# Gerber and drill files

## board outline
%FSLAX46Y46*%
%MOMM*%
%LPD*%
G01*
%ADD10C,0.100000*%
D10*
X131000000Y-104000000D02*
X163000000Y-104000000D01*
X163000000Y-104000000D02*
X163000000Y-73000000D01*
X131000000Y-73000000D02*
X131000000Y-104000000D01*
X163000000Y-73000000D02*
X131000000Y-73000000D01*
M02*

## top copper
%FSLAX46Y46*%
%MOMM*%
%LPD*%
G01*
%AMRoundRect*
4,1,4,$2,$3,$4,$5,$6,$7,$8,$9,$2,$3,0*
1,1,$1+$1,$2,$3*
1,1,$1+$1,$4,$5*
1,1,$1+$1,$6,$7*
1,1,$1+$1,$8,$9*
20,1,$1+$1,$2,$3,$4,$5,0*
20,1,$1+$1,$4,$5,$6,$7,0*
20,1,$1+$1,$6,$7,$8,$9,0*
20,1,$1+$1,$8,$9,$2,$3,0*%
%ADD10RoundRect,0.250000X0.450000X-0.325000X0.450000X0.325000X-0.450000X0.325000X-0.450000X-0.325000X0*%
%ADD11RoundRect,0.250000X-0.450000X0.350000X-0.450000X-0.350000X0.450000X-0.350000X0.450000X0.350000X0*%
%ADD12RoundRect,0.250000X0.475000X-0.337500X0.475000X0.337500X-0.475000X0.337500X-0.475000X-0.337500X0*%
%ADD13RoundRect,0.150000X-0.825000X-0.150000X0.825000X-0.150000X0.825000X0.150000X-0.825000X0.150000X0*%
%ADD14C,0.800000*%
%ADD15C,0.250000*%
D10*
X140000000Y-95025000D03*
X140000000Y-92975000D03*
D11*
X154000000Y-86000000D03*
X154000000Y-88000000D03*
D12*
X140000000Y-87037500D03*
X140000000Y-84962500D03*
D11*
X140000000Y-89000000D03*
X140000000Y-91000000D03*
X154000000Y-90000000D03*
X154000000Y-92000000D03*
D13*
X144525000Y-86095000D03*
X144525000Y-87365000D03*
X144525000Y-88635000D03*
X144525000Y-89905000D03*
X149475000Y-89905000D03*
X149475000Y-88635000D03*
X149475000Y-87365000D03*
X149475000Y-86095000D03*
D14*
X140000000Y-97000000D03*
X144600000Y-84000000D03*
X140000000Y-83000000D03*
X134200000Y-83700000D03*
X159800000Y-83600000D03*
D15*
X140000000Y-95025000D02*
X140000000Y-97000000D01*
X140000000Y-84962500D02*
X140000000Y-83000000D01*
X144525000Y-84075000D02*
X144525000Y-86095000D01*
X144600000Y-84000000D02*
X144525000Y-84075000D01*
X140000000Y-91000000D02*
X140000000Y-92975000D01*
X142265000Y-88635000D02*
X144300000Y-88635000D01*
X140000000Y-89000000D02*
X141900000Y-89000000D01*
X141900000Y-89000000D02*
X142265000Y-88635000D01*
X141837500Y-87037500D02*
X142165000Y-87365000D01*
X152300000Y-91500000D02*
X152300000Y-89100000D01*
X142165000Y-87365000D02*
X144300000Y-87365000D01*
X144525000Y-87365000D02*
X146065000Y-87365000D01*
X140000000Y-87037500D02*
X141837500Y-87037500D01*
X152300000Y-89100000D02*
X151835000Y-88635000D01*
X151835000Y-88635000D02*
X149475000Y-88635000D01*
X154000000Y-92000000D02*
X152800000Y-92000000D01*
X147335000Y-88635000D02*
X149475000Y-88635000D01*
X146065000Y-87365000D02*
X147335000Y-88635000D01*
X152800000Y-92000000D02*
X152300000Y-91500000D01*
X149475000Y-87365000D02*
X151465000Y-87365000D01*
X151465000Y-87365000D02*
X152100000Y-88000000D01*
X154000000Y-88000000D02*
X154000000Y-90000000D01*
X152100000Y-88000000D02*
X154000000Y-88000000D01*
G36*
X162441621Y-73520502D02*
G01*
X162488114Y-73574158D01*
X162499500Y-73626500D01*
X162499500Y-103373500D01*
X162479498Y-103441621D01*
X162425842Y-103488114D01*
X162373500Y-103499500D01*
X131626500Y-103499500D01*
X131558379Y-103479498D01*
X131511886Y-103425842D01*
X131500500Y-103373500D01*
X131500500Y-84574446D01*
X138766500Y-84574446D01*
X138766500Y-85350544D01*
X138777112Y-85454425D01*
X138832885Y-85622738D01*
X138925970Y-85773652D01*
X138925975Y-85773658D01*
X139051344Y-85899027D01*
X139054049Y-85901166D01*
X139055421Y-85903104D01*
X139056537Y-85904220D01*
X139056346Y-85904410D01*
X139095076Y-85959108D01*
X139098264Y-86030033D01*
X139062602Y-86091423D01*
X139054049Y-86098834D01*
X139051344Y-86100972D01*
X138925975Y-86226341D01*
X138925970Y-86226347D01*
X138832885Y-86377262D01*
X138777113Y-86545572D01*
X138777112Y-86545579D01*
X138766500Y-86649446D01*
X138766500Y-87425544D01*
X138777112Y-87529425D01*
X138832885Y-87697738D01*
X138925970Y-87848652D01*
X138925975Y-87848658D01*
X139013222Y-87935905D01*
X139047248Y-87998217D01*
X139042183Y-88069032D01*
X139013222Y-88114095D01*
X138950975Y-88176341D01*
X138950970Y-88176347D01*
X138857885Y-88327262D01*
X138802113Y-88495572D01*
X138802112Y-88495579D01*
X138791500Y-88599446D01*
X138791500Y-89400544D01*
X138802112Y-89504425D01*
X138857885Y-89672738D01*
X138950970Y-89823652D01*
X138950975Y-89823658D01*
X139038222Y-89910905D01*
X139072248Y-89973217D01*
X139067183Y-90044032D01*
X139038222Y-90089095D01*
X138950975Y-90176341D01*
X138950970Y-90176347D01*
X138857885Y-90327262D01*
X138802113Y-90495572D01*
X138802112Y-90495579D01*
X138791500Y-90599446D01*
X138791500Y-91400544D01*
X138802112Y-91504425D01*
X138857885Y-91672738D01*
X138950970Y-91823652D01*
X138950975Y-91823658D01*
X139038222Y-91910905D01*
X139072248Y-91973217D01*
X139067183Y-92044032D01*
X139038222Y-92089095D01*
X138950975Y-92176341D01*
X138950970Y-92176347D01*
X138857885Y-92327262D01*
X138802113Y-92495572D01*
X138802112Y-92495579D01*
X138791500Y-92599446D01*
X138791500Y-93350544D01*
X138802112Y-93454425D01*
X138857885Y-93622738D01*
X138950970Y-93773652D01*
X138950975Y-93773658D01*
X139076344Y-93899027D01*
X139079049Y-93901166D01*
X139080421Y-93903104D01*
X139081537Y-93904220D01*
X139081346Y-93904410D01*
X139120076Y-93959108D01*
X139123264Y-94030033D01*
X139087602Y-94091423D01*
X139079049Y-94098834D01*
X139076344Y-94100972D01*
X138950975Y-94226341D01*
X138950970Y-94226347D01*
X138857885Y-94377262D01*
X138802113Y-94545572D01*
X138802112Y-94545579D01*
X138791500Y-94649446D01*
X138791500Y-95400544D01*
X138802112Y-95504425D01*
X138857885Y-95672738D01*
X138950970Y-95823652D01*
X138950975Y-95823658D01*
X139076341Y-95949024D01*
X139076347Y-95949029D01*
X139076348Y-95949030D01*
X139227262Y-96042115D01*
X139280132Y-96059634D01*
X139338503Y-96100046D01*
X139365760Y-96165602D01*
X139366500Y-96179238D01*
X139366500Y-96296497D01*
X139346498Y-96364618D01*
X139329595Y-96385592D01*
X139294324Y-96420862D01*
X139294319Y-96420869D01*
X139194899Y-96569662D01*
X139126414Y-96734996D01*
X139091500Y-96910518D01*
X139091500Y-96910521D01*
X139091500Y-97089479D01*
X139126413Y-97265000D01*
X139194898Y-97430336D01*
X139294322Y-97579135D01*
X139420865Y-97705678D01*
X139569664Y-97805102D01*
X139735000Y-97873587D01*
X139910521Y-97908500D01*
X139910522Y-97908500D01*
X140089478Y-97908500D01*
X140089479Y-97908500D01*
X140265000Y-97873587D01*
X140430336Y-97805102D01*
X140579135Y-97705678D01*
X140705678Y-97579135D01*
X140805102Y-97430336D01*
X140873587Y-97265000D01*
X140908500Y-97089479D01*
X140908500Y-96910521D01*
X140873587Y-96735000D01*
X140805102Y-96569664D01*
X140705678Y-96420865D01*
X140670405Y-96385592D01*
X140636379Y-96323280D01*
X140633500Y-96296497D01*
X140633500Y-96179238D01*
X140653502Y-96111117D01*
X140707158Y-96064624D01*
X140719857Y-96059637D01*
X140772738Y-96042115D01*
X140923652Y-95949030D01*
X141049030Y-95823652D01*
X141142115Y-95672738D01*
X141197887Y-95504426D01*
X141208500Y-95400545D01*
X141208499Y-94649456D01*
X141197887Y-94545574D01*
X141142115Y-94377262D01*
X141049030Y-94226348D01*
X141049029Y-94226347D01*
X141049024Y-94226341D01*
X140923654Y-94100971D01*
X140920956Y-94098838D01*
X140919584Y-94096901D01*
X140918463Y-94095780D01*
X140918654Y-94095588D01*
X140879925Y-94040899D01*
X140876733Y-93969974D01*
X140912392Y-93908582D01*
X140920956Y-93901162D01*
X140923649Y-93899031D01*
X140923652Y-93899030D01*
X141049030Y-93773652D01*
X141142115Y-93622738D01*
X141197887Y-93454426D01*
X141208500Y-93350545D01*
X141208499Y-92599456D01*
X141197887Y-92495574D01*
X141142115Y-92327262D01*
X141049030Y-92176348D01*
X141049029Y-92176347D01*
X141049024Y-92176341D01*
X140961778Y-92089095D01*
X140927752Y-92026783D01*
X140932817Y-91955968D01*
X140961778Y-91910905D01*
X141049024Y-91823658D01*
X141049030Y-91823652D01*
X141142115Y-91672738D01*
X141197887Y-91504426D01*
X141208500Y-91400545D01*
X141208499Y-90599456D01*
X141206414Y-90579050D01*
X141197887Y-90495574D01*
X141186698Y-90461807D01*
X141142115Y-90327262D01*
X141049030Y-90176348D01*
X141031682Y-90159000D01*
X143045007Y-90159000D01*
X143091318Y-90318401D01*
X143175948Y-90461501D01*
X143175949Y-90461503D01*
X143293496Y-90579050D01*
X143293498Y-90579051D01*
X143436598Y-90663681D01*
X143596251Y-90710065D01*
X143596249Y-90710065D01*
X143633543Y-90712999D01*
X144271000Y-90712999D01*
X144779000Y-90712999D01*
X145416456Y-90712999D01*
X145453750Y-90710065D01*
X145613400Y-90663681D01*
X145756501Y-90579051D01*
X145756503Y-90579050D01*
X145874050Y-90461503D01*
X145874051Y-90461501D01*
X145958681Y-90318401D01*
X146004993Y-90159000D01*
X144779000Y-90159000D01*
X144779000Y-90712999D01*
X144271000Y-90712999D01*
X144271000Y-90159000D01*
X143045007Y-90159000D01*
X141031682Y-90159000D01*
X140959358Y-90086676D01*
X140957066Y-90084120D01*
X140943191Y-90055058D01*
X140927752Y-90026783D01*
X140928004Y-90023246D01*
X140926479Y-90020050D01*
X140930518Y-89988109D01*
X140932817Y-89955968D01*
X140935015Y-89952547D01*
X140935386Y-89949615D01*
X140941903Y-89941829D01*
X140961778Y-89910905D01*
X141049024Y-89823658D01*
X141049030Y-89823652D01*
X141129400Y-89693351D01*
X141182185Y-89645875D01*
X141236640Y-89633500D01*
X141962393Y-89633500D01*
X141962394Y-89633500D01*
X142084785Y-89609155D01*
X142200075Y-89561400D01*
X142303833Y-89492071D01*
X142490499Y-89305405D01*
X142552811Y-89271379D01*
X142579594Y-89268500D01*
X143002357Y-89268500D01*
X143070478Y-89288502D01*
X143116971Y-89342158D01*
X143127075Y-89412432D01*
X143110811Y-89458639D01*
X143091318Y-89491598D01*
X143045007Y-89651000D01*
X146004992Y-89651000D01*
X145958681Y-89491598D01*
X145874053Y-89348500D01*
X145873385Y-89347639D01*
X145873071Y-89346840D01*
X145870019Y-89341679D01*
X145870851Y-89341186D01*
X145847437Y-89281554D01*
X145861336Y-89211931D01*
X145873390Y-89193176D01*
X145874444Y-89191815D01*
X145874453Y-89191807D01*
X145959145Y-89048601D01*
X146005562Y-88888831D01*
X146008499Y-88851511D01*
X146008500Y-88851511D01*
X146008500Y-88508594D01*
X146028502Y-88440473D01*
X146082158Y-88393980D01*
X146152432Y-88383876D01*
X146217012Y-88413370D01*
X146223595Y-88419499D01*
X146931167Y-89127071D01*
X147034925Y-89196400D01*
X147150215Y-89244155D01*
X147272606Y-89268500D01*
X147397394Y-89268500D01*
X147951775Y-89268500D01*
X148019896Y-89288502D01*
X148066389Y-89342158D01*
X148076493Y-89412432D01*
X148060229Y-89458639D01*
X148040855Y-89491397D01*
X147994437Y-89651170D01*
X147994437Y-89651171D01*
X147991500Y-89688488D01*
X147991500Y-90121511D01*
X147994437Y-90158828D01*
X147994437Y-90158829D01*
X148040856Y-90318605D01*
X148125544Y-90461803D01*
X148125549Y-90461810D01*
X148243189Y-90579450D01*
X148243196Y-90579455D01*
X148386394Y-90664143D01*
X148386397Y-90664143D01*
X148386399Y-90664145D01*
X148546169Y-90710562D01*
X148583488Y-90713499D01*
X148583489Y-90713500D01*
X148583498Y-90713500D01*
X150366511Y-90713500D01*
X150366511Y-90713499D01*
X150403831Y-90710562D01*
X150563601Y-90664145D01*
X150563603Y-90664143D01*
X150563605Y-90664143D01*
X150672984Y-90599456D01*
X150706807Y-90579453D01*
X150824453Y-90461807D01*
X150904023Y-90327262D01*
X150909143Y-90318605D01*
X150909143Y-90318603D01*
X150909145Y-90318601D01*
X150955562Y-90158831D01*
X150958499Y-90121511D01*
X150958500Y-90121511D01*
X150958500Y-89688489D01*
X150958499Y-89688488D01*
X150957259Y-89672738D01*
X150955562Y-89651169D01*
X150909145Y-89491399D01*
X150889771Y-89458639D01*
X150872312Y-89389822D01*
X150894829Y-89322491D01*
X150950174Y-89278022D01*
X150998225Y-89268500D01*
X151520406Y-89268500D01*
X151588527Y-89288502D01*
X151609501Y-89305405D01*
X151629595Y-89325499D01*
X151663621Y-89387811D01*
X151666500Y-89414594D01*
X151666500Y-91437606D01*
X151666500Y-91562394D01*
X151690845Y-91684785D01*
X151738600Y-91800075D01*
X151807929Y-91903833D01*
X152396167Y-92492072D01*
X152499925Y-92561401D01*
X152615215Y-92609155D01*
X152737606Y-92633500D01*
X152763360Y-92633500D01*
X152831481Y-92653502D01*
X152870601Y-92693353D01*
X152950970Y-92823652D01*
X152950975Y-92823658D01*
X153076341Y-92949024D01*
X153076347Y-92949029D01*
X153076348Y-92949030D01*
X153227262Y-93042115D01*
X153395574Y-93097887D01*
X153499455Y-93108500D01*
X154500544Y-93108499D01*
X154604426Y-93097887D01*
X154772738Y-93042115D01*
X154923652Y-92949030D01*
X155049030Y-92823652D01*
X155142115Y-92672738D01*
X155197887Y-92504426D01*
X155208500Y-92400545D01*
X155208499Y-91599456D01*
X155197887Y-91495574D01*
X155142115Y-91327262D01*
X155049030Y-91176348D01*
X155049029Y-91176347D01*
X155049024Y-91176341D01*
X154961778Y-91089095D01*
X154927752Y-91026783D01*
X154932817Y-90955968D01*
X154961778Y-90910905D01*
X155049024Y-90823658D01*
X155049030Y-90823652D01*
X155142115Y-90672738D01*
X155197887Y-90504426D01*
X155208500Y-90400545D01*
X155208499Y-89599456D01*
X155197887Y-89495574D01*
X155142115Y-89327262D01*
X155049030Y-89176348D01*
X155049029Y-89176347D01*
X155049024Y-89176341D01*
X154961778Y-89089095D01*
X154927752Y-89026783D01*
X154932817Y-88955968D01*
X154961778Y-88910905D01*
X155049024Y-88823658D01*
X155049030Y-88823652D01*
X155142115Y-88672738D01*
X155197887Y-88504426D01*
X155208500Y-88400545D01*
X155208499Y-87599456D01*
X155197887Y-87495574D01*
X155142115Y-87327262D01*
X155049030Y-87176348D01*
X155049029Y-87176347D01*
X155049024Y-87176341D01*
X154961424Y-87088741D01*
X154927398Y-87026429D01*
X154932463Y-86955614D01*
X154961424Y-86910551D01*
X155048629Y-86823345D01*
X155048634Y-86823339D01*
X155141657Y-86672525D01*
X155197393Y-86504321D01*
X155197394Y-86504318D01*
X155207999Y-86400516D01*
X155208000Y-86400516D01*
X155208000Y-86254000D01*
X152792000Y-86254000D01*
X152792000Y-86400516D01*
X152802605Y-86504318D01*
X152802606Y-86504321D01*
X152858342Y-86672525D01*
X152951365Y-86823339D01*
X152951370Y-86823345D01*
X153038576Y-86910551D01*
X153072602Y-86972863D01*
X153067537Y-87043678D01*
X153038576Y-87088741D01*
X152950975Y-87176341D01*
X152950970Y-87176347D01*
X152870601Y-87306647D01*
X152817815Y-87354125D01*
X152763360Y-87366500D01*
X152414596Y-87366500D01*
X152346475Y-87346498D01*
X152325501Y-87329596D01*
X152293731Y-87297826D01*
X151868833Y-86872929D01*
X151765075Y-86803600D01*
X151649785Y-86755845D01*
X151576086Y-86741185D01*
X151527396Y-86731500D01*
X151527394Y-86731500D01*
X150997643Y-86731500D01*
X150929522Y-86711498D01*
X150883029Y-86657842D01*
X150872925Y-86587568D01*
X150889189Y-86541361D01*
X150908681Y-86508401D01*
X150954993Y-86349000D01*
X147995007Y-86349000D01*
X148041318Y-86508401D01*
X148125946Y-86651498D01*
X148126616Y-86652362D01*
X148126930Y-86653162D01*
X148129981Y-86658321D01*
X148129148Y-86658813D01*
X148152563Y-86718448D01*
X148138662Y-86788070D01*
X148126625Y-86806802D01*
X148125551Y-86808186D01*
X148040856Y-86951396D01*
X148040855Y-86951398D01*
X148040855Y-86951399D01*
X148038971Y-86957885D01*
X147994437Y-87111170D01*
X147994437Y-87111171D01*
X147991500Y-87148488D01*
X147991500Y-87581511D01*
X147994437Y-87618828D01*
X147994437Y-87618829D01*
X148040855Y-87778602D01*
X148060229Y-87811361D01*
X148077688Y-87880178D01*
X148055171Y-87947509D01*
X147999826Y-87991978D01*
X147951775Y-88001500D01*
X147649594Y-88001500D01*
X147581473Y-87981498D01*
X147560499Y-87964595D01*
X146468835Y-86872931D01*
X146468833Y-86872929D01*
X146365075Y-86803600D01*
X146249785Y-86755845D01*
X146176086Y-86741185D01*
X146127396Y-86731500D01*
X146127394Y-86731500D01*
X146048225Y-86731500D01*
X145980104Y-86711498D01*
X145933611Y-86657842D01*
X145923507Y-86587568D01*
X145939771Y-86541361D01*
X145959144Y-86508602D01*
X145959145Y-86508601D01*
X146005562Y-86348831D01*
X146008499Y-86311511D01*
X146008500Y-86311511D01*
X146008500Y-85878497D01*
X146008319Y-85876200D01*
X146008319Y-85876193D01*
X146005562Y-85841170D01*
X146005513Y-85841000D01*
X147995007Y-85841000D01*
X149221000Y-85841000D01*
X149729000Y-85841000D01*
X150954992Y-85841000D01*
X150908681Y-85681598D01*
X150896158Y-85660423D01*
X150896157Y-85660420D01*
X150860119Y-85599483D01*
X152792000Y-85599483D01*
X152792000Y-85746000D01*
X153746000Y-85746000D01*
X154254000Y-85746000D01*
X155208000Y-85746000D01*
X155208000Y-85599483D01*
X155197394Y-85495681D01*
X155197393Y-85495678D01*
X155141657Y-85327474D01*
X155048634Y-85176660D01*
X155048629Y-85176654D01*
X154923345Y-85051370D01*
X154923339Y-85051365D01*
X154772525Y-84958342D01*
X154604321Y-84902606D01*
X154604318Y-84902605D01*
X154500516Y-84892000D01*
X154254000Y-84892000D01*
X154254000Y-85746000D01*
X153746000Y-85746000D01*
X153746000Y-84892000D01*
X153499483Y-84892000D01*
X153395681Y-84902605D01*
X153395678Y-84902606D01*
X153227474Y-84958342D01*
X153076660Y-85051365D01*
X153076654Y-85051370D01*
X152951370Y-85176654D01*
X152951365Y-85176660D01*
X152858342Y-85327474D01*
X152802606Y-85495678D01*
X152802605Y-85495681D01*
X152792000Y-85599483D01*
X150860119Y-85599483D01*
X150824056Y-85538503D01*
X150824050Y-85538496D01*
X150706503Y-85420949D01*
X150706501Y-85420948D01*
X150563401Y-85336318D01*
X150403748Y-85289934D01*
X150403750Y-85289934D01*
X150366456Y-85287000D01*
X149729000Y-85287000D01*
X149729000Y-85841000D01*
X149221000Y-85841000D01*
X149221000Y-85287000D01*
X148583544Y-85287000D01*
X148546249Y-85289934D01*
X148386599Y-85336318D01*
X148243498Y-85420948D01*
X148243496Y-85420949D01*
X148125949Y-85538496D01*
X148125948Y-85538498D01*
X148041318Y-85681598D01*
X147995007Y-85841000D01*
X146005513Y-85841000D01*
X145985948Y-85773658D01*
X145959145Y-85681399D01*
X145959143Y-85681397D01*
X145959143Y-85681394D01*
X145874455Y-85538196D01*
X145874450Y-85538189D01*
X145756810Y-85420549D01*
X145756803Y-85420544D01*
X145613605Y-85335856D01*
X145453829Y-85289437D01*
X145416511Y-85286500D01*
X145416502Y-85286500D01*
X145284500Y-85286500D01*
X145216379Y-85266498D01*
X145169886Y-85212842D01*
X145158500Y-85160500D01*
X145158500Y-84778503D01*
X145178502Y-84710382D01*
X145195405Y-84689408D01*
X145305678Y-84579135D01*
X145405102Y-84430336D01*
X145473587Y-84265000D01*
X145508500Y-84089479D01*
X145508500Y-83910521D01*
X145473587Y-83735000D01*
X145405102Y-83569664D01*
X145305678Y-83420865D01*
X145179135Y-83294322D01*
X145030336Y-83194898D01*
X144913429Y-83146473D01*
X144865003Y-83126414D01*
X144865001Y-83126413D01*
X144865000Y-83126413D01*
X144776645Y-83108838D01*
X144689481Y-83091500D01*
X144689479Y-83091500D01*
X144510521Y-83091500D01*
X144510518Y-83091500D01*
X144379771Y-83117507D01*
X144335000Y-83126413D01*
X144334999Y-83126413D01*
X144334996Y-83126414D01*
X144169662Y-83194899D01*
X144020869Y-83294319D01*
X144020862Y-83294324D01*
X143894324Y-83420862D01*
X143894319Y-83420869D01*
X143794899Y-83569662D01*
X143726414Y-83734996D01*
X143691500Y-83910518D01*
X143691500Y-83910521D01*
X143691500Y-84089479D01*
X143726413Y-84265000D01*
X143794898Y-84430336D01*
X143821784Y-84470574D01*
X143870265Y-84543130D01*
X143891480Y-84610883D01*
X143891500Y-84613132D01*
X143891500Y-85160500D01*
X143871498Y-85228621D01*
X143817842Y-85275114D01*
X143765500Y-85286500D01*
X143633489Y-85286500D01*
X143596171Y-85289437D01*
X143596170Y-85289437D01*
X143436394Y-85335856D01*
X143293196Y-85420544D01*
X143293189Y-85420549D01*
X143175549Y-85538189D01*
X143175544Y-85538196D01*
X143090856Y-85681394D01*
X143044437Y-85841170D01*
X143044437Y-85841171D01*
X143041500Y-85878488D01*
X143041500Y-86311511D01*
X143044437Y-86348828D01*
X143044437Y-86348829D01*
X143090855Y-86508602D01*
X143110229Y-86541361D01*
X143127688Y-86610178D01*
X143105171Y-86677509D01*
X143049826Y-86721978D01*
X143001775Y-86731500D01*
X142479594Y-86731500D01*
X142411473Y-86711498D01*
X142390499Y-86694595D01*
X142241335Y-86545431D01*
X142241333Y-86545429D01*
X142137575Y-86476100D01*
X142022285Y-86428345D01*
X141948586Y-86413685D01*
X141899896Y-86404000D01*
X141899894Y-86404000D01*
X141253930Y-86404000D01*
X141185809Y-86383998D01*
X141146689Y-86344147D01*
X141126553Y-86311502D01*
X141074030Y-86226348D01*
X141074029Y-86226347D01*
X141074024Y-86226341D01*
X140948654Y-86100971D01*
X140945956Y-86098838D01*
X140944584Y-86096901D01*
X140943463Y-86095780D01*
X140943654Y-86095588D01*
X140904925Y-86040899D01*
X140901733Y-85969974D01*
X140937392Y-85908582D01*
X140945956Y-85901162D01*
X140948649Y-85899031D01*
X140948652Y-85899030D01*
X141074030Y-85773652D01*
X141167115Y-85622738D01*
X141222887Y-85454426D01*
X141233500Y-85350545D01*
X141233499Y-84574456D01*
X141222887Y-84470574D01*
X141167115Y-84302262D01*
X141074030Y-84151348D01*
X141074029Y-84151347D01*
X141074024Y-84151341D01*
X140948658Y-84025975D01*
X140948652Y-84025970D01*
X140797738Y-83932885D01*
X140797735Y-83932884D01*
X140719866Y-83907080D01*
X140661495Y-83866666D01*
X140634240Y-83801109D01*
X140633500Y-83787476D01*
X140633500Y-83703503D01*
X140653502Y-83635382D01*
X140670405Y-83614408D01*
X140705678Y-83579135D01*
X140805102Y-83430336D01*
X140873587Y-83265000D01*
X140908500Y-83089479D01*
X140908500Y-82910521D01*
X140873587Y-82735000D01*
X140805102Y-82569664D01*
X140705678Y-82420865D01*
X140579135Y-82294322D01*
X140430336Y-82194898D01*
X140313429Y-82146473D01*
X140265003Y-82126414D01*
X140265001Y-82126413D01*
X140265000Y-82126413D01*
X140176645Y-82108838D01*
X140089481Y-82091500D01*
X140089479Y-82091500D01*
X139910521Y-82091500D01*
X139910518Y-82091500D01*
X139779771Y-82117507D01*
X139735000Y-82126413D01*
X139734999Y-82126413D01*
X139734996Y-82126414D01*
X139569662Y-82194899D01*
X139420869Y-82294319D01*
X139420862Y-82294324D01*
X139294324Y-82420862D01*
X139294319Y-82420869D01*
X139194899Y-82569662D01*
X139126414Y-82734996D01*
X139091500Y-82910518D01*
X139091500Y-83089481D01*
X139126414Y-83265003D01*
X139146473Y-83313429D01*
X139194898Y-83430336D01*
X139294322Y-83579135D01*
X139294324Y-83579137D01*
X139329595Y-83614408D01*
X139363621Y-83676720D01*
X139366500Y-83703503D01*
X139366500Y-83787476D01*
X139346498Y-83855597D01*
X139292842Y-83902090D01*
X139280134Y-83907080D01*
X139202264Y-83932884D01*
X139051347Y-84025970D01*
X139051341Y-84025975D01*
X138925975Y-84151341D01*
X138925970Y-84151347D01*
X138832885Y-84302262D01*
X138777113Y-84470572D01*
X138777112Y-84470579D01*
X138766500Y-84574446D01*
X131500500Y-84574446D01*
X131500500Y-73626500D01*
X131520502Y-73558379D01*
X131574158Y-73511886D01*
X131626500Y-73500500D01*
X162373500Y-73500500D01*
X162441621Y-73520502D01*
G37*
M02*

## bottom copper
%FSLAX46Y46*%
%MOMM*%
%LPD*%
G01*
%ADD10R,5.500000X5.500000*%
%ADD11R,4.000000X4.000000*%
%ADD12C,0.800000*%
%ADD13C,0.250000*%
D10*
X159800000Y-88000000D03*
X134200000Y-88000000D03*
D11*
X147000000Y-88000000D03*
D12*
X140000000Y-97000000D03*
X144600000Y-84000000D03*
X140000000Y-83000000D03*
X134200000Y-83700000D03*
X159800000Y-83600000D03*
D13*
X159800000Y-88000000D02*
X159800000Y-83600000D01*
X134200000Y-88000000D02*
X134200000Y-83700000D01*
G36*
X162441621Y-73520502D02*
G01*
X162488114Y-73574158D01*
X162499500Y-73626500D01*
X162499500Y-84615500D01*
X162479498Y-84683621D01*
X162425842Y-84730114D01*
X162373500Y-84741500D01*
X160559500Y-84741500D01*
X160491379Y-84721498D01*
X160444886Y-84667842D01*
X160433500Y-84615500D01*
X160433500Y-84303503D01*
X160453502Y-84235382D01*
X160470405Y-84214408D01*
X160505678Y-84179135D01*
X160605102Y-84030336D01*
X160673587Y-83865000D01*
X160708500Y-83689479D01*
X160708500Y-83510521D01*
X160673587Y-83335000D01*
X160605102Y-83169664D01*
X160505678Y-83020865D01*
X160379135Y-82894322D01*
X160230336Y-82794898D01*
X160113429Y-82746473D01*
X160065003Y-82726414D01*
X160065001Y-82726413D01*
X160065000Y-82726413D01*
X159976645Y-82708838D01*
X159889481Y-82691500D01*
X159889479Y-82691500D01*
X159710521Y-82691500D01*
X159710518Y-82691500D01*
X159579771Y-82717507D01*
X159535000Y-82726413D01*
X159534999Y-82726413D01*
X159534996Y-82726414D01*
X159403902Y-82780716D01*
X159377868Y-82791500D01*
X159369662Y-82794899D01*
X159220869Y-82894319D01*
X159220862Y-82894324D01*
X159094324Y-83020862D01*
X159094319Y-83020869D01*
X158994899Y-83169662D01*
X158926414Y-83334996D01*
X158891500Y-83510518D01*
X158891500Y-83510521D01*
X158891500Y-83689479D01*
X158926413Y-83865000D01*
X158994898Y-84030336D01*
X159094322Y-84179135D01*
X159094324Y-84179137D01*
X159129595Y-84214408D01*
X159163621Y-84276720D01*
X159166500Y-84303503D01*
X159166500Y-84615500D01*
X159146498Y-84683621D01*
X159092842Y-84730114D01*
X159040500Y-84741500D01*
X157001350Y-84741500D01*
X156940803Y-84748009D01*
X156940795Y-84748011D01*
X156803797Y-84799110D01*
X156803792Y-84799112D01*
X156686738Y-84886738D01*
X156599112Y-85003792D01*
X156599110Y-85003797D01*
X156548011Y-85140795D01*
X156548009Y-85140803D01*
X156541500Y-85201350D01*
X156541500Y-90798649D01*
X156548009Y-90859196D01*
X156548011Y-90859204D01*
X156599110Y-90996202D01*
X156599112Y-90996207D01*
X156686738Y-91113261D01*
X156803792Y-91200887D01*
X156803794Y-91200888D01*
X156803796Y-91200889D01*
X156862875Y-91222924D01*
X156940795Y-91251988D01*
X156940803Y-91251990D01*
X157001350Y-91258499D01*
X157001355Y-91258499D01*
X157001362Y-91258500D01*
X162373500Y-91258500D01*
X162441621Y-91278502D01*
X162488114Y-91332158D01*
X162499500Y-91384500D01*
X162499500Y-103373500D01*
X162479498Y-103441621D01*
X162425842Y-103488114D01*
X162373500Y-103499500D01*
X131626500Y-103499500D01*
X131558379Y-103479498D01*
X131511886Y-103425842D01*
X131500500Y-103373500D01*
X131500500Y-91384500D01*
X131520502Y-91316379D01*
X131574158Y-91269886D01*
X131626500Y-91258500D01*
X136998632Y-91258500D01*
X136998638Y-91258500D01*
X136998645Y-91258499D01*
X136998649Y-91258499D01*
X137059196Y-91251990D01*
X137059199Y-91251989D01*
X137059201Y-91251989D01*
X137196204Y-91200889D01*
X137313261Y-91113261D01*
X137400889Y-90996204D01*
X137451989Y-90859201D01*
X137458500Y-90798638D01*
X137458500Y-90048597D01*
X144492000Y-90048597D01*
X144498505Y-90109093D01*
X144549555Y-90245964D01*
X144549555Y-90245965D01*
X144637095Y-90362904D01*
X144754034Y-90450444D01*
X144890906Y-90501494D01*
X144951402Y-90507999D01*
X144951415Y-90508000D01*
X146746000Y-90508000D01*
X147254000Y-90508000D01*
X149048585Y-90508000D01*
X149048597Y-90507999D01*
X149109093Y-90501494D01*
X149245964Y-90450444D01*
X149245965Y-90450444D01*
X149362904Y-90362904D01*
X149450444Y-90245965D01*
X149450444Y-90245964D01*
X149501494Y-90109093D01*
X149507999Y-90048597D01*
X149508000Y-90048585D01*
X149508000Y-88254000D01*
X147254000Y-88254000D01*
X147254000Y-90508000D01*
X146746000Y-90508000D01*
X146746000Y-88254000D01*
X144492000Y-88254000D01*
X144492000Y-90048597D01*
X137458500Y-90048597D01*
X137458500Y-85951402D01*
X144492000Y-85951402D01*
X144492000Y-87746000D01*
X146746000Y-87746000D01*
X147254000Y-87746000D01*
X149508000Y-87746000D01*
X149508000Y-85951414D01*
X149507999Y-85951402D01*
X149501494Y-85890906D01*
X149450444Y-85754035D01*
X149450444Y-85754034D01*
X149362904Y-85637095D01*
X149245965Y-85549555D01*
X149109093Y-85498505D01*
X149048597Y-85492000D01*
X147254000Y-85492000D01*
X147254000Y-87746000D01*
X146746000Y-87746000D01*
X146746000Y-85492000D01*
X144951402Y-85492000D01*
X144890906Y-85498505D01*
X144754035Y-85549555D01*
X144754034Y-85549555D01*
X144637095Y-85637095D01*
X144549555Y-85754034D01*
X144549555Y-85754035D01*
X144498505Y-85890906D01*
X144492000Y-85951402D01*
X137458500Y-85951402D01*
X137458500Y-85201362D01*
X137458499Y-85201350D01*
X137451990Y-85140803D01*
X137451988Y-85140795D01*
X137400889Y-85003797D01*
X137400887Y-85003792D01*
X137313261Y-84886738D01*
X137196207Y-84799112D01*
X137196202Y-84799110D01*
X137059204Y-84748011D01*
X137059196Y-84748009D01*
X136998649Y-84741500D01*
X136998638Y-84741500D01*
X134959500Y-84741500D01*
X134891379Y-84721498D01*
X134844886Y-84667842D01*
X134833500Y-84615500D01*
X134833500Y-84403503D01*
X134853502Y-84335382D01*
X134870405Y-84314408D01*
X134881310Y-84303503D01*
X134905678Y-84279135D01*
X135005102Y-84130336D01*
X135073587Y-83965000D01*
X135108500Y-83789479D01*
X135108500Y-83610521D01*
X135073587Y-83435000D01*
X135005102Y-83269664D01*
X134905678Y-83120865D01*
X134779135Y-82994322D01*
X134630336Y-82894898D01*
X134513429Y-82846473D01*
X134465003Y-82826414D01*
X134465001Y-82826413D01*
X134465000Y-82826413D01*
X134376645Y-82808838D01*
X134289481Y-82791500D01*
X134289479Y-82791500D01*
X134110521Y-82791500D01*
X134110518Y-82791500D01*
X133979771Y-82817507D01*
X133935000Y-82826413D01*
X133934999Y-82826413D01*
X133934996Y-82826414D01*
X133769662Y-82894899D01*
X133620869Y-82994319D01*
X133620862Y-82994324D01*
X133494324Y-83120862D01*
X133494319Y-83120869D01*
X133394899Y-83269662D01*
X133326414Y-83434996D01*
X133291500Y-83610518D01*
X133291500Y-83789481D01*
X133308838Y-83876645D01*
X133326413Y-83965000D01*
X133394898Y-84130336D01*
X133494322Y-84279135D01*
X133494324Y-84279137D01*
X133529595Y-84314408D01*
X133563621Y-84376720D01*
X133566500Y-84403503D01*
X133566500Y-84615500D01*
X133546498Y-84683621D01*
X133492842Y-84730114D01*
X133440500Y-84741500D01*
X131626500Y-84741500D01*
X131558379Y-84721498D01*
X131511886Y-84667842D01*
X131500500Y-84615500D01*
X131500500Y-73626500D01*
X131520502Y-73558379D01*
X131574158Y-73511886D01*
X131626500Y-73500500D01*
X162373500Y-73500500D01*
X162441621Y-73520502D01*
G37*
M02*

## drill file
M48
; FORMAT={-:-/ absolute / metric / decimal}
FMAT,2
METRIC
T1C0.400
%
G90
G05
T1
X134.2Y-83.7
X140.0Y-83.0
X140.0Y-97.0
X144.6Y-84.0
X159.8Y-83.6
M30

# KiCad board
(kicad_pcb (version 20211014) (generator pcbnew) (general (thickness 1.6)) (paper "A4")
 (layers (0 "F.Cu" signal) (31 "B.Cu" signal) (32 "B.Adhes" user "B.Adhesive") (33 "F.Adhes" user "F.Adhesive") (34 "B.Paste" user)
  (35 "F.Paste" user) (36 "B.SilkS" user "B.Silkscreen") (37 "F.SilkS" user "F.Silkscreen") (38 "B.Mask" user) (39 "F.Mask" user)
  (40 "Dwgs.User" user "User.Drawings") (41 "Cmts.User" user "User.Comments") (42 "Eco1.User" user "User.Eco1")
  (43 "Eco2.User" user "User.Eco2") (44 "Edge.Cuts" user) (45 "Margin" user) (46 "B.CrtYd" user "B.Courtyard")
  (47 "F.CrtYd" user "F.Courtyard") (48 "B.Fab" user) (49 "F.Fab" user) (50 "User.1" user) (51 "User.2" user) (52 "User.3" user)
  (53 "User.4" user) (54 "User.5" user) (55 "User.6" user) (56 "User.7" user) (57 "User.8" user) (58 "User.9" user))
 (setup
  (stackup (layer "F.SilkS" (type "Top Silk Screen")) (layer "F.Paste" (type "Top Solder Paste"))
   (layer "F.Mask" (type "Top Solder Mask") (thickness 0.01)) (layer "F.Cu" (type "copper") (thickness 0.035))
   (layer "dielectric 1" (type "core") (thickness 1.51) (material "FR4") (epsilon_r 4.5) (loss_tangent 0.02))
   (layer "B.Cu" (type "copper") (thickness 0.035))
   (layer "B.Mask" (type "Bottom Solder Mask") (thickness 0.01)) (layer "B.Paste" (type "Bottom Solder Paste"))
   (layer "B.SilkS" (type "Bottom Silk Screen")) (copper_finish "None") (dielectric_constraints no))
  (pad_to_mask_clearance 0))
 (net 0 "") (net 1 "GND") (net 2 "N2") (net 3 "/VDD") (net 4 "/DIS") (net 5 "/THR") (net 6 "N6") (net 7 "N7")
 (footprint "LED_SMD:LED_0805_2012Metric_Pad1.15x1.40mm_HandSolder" (layer "F.Cu") (at 140 94 90)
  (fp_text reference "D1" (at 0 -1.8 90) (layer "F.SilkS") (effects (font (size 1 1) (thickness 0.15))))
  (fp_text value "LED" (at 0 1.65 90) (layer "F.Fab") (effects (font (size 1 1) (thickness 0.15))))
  (pad "1" smd roundrect (at -1.025 0 90) (size 1.15 1.4) (layers "F.Cu" "F.Paste" "F.Mask") (roundrect_rratio 0.217391) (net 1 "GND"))
  (pad "2" smd roundrect (at 1.025 0 90) (size 1.15 1.4) (layers "F.Cu" "F.Paste" "F.Mask") (roundrect_rratio 0.217391) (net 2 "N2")))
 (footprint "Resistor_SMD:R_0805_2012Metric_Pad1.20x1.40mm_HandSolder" (layer "F.Cu") (at 154 87 -90)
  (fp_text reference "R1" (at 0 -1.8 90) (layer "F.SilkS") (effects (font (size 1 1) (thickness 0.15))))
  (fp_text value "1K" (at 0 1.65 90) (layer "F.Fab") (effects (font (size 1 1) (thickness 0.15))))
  (pad "1" smd roundrect (at -1 0 270) (size 1.2 1.4) (layers "F.Cu" "F.Paste" "F.Mask") (roundrect_rratio 0.208333) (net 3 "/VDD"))
  (pad "2" smd roundrect (at 1 0 270) (size 1.2 1.4) (layers "F.Cu" "F.Paste" "F.Mask") (roundrect_rratio 0.208333) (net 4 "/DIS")))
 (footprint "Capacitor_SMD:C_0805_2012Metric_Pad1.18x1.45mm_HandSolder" (layer "F.Cu") (at 140 86 90)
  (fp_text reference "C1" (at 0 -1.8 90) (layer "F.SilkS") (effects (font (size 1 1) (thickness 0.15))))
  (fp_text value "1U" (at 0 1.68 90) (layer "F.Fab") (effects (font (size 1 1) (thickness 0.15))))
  (pad "1" smd roundrect (at -1.0375 0 90) (size 1.175 1.45) (layers "F.Cu" "F.Paste" "F.Mask") (roundrect_rratio 0.212766) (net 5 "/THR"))
  (pad "2" smd roundrect (at 1.0375 0 90) (size 1.175 1.45) (layers "F.Cu" "F.Paste" "F.Mask") (roundrect_rratio 0.212766) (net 1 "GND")))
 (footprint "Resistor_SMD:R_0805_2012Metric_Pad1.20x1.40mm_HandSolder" (layer "F.Cu") (at 140 90 -90)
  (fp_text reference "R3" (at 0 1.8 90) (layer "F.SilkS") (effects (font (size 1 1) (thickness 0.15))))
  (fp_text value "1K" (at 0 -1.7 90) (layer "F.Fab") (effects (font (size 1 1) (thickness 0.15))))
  (pad "1" smd roundrect (at -1 0 270) (size 1.2 1.4) (layers "F.Cu" "F.Paste" "F.Mask") (roundrect_rratio 0.208333) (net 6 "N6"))
  (pad "2" smd roundrect (at 1 0 270) (size 1.2 1.4) (layers "F.Cu" "F.Paste" "F.Mask") (roundrect_rratio 0.208333) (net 2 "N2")))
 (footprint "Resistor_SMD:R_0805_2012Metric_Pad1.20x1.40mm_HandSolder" (layer "F.Cu") (at 154 91 -90)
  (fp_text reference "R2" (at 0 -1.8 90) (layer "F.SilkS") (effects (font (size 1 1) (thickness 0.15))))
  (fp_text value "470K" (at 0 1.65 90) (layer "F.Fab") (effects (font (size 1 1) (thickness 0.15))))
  (pad "1" smd roundrect (at -1 0 270) (size 1.2 1.4) (layers "F.Cu" "F.Paste" "F.Mask") (roundrect_rratio 0.208333) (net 4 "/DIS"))
  (pad "2" smd roundrect (at 1 0 270) (size 1.2 1.4) (layers "F.Cu" "F.Paste" "F.Mask") (roundrect_rratio 0.208333) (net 5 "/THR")))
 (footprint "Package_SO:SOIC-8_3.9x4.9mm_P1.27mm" (layer "F.Cu") (at 147 88)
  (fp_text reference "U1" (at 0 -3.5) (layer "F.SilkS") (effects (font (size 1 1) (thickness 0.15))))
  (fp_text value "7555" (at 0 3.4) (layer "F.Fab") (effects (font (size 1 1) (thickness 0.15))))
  (pad "1" smd roundrect (at -2.475 -1.905) (size 1.95 0.6) (layers "F.Cu" "F.Paste" "F.Mask") (roundrect_rratio 0.25) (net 1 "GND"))
  (pad "2" smd roundrect (at -2.475 -0.635) (size 1.95 0.6) (layers "F.Cu" "F.Paste" "F.Mask") (roundrect_rratio 0.25) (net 5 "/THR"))
  (pad "3" smd roundrect (at -2.475 0.635) (size 1.95 0.6) (layers "F.Cu" "F.Paste" "F.Mask") (roundrect_rratio 0.25) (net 6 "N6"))
  (pad "4" smd roundrect (at -2.475 1.905) (size 1.95 0.6) (layers "F.Cu" "F.Paste" "F.Mask") (roundrect_rratio 0.25) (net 3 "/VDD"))
  (pad "5" smd roundrect (at 2.475 1.905) (size 1.95 0.6) (layers "F.Cu" "F.Paste" "F.Mask") (roundrect_rratio 0.25) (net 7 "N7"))
  (pad "6" smd roundrect (at 2.475 0.635) (size 1.95 0.6) (layers "F.Cu" "F.Paste" "F.Mask") (roundrect_rratio 0.25) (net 5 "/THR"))
  (pad "7" smd roundrect (at 2.475 -0.635) (size 1.95 0.6) (layers "F.Cu" "F.Paste" "F.Mask") (roundrect_rratio 0.25) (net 4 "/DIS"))
  (pad "8" smd roundrect (at 2.475 -1.905) (size 1.95 0.6) (layers "F.Cu" "F.Paste" "F.Mask") (roundrect_rratio 0.25) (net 3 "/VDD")))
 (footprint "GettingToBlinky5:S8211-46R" (layer "B.Cu") (at 147 88 180)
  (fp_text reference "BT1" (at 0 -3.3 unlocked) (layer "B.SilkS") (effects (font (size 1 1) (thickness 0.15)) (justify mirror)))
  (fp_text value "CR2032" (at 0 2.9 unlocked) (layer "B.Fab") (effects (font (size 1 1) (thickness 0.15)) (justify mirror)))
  (pad "1" smd rect (at -12.8 0 180) (size 5.5 5.5) (layers "B.Cu" "B.Paste" "B.Mask") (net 3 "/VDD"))
  (pad "1" smd rect (at 12.8 0 180) (size 5.5 5.5) (layers "B.Cu" "B.Paste" "B.Mask") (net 3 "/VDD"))
  (pad "2" smd rect (at 0 0 180) (size 4 4) (layers "B.Cu" "B.Paste" "B.Mask") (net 1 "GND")))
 (gr_line (start 131 104) (end 163 104) (layer "Edge.Cuts") (width 0.1))
 (gr_line (start 163 104) (end 163 73) (layer "Edge.Cuts") (width 0.1))
 (gr_line (start 131 73) (end 131 104) (layer "Edge.Cuts") (width 0.1))
 (gr_line (start 163 73) (end 131 73) (layer "Edge.Cuts") (width 0.1))
 (segment (start 140 95.025) (end 140 97) (width 0.25) (layer "F.Cu") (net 1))
 (segment (start 140 84.9625) (end 140 83) (width 0.25) (layer "F.Cu") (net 1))
 (segment (start 144.525 84.075) (end 144.525 86.095) (width 0.25) (layer "F.Cu") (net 1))
 (segment (start 144.6 84) (end 144.525 84.075) (width 0.25) (layer "F.Cu") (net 1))
 (via (at 140 97) (size 0.8) (drill 0.4) (layers "F.Cu" "B.Cu") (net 1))
 (via (at 144.6 84) (size 0.8) (drill 0.4) (layers "F.Cu" "B.Cu") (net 1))
 (via (at 140 83) (size 0.8) (drill 0.4) (layers "F.Cu" "B.Cu") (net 1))
 (segment (start 140 91) (end 140 92.975) (width 0.25) (layer "F.Cu") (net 2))
 (segment (start 142.265 88.635) (end 144.3 88.635) (width 0.25) (layer "F.Cu") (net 6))
 (segment (start 140 89) (end 141.9 89) (width 0.25) (layer "F.Cu") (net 6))
 (segment (start 141.9 89) (end 142.265 88.635) (width 0.25) (layer "F.Cu") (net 6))
 (via (at 134.2 83.7) (size 0.8) (drill 0.4) (layers "F.Cu" "B.Cu") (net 3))
 (via (at 159.8 83.6) (size 0.8) (drill 0.4) (layers "F.Cu" "B.Cu") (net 3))
 (segment (start 159.8 88) (end 159.8 83.6) (width 0.25) (layer "B.Cu") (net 3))
 (segment (start 134.2 88) (end 134.2 83.7) (width 0.25) (layer "B.Cu") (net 3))
 (segment (start 141.8375 87.0375) (end 142.165 87.365) (width 0.25) (layer "F.Cu") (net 5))
 (segment (start 152.3 91.5) (end 152.3 89.1) (width 0.25) (layer "F.Cu") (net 5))
 (segment (start 142.165 87.365) (end 144.3 87.365) (width 0.25) (layer "F.Cu") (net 5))
 (segment (start 144.525 87.365) (end 146.065 87.365) (width 0.25) (layer "F.Cu") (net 5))
 (segment (start 140 87.0375) (end 141.8375 87.0375) (width 0.25) (layer "F.Cu") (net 5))
 (segment (start 152.3 89.1) (end 151.835 88.635) (width 0.25) (layer "F.Cu") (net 5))
 (segment (start 151.835 88.635) (end 149.475 88.635) (width 0.25) (layer "F.Cu") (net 5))
 (segment (start 154 92) (end 152.8 92) (width 0.25) (layer "F.Cu") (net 5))
 (segment (start 147.335 88.635) (end 149.475 88.635) (width 0.25) (layer "F.Cu") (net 5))
 (segment (start 146.065 87.365) (end 147.335 88.635) (width 0.25) (layer "F.Cu") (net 5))
 (segment (start 152.8 92) (end 152.3 91.5) (width 0.25) (layer "F.Cu") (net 5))
 (segment (start 149.475 87.365) (end 151.465 87.365) (width 0.25) (layer "F.Cu") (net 4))
 (segment (start 151.465 87.365) (end 152.1 88) (width 0.25) (layer "F.Cu") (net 4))
 (segment (start 154 88) (end 154 90) (width 0.25) (layer "F.Cu") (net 4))
 (segment (start 152.1 88) (end 154 88) (width 0.25) (layer "F.Cu") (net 4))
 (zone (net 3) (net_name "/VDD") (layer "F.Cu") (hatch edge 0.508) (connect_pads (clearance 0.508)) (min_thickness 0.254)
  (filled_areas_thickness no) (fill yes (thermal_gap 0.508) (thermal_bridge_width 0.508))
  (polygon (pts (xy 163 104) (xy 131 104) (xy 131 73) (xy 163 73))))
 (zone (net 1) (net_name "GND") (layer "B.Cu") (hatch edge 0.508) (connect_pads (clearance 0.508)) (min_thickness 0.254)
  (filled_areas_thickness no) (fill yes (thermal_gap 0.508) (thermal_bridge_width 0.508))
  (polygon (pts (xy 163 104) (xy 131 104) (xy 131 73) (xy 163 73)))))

